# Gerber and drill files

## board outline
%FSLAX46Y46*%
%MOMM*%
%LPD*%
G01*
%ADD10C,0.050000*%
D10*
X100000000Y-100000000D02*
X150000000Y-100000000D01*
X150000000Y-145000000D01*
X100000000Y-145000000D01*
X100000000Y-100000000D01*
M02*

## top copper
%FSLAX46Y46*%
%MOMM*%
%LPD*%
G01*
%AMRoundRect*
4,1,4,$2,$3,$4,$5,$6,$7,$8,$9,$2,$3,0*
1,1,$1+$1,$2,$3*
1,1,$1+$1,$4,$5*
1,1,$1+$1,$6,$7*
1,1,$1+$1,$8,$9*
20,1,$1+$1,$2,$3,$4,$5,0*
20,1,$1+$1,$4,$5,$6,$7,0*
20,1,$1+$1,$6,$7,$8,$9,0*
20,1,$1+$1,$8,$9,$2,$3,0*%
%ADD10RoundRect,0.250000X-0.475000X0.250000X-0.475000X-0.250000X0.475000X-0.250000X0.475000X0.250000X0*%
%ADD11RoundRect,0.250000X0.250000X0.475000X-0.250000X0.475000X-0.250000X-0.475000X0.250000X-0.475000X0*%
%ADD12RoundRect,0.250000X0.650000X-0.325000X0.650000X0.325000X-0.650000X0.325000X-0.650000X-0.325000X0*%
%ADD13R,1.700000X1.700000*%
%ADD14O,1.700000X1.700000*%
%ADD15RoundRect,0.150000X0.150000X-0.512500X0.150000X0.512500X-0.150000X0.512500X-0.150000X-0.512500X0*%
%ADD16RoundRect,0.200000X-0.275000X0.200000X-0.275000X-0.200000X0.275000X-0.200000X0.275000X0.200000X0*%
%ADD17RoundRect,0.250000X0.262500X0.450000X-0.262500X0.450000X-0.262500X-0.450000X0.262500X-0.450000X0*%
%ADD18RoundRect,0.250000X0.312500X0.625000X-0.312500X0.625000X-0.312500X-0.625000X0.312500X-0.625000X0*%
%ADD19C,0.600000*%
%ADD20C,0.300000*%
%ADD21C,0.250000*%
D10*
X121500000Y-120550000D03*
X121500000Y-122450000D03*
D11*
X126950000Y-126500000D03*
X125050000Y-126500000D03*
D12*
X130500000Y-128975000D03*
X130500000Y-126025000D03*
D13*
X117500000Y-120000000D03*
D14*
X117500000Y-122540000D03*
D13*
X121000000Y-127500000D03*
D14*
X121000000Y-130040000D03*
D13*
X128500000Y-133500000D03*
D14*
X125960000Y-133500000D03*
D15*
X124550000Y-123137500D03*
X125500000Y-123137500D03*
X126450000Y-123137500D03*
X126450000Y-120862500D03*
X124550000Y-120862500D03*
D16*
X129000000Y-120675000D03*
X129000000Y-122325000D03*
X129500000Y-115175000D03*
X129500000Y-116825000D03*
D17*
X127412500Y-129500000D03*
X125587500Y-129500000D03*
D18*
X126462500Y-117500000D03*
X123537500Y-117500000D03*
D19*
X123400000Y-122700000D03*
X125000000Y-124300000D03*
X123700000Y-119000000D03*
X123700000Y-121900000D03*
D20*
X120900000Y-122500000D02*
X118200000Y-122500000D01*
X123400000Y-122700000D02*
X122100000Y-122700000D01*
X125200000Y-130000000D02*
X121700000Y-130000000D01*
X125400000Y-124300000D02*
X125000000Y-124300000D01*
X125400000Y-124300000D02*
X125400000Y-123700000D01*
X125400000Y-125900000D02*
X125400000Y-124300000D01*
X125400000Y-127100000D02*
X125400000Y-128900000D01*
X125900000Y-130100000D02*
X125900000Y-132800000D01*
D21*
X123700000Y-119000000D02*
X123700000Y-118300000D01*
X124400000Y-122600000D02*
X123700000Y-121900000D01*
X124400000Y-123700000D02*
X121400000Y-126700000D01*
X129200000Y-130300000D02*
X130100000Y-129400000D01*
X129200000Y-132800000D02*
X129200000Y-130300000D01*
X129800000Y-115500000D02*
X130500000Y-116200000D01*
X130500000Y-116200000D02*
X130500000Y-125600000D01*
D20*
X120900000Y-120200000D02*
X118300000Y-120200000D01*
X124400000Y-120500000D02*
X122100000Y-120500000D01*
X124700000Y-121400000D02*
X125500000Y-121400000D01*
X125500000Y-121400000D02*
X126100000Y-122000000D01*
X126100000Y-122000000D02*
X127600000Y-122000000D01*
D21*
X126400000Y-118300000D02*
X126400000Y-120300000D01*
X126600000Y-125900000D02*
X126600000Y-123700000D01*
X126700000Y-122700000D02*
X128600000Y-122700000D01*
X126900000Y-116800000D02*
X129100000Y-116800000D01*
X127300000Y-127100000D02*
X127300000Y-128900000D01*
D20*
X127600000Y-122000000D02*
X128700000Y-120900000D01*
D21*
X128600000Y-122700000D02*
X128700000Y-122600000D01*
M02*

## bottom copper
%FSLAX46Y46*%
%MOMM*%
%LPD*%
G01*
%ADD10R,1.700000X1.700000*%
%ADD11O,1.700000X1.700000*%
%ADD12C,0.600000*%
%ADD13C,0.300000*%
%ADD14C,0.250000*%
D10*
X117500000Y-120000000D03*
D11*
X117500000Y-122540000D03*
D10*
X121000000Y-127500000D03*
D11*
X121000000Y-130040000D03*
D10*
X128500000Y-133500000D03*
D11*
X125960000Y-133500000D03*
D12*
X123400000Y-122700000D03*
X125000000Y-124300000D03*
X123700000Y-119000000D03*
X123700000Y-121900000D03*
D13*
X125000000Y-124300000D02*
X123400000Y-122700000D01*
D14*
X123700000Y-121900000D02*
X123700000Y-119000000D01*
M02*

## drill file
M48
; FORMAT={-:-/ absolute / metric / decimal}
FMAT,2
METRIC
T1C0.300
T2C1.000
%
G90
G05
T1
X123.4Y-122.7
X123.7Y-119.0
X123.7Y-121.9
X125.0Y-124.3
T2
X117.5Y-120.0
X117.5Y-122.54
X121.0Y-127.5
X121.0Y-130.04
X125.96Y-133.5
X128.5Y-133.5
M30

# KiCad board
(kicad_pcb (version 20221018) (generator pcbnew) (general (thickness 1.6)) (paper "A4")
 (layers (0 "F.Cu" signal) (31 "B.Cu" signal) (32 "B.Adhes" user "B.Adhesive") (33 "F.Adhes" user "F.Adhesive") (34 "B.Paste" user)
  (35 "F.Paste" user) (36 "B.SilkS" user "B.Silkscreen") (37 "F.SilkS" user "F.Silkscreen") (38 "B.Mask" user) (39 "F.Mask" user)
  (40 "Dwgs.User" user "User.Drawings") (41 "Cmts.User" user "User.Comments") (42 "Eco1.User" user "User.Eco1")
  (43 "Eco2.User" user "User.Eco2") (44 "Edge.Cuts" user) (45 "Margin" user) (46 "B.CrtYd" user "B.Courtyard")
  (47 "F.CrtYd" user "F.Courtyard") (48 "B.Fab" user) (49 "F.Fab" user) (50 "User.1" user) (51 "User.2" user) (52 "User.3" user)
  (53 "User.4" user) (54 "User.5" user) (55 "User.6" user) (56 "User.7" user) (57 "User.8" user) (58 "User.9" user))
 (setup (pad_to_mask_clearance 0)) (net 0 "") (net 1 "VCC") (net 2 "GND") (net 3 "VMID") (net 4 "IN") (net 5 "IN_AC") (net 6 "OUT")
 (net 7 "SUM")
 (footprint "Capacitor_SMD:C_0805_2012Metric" (layer "F.Cu") (at 121.5 121.5 -90)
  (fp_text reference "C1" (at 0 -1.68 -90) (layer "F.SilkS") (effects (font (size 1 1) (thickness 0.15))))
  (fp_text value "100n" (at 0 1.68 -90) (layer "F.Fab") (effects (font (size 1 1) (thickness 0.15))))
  (pad "1" smd roundrect (at -0.95 0 270) (size 1 1.45) (layers "F.Cu" "F.Paste" "F.Mask") (roundrect_rratio 0.25) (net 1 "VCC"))
  (pad "2" smd roundrect (at 0.95 0 270) (size 1 1.45) (layers "F.Cu" "F.Paste" "F.Mask") (roundrect_rratio 0.25) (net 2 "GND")))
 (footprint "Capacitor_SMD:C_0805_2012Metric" (layer "F.Cu") (at 126 126.5 180)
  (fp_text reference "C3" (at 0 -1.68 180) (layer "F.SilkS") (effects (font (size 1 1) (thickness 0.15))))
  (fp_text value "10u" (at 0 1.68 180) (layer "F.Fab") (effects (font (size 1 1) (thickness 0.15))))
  (pad "1" smd roundrect (at -0.95 0 180) (size 1 1.45) (layers "F.Cu" "F.Paste" "F.Mask") (roundrect_rratio 0.25) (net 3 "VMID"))
  (pad "2" smd roundrect (at 0.95 0 180) (size 1 1.45) (layers "F.Cu" "F.Paste" "F.Mask") (roundrect_rratio 0.25) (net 2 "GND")))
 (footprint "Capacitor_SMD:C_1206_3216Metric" (layer "F.Cu") (at 130.5 127.5 90)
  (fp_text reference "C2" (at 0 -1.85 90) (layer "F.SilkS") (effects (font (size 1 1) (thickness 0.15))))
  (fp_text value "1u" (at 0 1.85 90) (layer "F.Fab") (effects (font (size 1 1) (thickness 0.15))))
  (pad "1" smd roundrect (at -1.475 0 90) (size 1.15 1.8) (layers "F.Cu" "F.Paste" "F.Mask") (roundrect_rratio 0.217391) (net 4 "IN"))
  (pad "2" smd roundrect (at 1.475 0 90) (size 1.15 1.8) (layers "F.Cu" "F.Paste" "F.Mask") (roundrect_rratio 0.217391) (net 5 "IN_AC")))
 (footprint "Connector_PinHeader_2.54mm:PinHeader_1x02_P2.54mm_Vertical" (layer "F.Cu") (at 117.5 120)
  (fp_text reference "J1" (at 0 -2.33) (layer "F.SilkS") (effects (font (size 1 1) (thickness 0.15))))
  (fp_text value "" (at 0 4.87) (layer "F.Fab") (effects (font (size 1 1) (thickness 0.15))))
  (pad "1" thru_hole rect (at 0 0) (size 1.7 1.7) (drill 1) (layers "*.Cu" "*.Mask") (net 1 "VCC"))
  (pad "2" thru_hole oval (at 0 2.54) (size 1.7 1.7) (drill 1) (layers "*.Cu" "*.Mask") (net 2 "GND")))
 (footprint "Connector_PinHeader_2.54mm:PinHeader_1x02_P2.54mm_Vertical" (layer "F.Cu") (at 121 127.5)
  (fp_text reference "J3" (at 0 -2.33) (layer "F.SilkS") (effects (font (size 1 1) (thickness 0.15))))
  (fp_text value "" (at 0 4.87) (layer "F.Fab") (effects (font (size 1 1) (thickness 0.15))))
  (pad "1" thru_hole rect (at 0 0) (size 1.7 1.7) (drill 1) (layers "*.Cu" "*.Mask") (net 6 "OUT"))
  (pad "2" thru_hole oval (at 0 2.54) (size 1.7 1.7) (drill 1) (layers "*.Cu" "*.Mask") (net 2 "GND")))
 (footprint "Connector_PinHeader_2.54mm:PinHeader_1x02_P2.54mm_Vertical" (layer "F.Cu") (at 128.5 133.5 -90)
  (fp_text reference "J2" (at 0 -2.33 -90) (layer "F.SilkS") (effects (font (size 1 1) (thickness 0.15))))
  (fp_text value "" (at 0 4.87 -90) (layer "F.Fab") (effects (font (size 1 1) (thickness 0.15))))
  (pad "1" thru_hole rect (at 0 0 270) (size 1.7 1.7) (drill 1) (layers "*.Cu" "*.Mask") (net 4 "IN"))
  (pad "2" thru_hole oval (at 0 2.54 270) (size 1.7 1.7) (drill 1) (layers "*.Cu" "*.Mask") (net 2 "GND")))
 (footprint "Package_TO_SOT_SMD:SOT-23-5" (layer "F.Cu") (at 125.5 122 90)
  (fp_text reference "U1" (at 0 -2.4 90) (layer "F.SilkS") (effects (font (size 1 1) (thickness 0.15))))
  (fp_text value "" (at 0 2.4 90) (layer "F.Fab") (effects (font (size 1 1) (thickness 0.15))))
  (pad "1" smd roundrect (at -1.1375 -0.95 90) (size 1.325 0.6) (layers "F.Cu" "F.Paste" "F.Mask") (roundrect_rratio 0.25) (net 6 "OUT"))
  (pad "2" smd roundrect (at -1.1375 0 90) (size 1.325 0.6) (layers "F.Cu" "F.Paste" "F.Mask") (roundrect_rratio 0.25) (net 2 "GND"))
  (pad "3" smd roundrect (at -1.1375 0.95 90) (size 1.325 0.6) (layers "F.Cu" "F.Paste" "F.Mask") (roundrect_rratio 0.25) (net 3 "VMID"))
  (pad "4" smd roundrect (at 1.1375 0.95 90) (size 1.325 0.6) (layers "F.Cu" "F.Paste" "F.Mask") (roundrect_rratio 0.25) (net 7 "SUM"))
  (pad "5" smd roundrect (at 1.1375 -0.95 90) (size 1.325 0.6) (layers "F.Cu" "F.Paste" "F.Mask") (roundrect_rratio 0.25) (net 1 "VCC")))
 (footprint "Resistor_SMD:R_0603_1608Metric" (layer "F.Cu") (at 129 121.5 -90)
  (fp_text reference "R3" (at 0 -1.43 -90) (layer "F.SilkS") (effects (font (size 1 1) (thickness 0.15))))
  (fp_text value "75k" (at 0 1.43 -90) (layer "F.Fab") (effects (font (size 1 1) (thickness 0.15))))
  (pad "1" smd roundrect (at -0.825 0 270) (size 0.8 0.95) (layers "F.Cu" "F.Paste" "F.Mask") (roundrect_rratio 0.25) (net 1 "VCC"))
  (pad "2" smd roundrect (at 0.825 0 270) (size 0.8 0.95) (layers "F.Cu" "F.Paste" "F.Mask") (roundrect_rratio 0.25) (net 3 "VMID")))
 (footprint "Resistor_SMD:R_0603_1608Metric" (layer "F.Cu") (at 129.5 116 -90)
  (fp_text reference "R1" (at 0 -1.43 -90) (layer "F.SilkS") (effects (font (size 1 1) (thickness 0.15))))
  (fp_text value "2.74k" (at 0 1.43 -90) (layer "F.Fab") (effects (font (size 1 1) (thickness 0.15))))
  (pad "1" smd roundrect (at -0.825 0 270) (size 0.8 0.95) (layers "F.Cu" "F.Paste" "F.Mask") (roundrect_rratio 0.25) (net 5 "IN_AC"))
  (pad "2" smd roundrect (at 0.825 0 270) (size 0.8 0.95) (layers "F.Cu" "F.Paste" "F.Mask") (roundrect_rratio 0.25) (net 7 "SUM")))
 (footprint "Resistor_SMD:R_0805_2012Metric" (layer "F.Cu") (at 126.5 129.5 180)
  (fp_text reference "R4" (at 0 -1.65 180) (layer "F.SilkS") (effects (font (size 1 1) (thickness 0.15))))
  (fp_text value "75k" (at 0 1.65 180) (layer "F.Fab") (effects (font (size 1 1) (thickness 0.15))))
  (pad "1" smd roundrect (at -0.9125 0 180) (size 1.025 1.4) (layers "F.Cu" "F.Paste" "F.Mask") (roundrect_rratio 0.243902) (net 3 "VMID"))
  (pad "2" smd roundrect (at 0.9125 0 180) (size 1.025 1.4) (layers "F.Cu" "F.Paste" "F.Mask") (roundrect_rratio 0.243902) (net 2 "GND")))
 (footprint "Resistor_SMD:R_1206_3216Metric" (layer "F.Cu") (at 125 117.5 180)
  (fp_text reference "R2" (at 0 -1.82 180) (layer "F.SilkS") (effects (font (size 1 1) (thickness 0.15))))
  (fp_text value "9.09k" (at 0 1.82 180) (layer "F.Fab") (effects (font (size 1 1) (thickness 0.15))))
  (pad "1" smd roundrect (at -1.4625 0 180) (size 1.125 1.75) (layers "F.Cu" "F.Paste" "F.Mask") (roundrect_rratio 0.222222) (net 7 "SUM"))
  (pad "2" smd roundrect (at 1.4625 0 180) (size 1.125 1.75) (layers "F.Cu" "F.Paste" "F.Mask") (roundrect_rratio 0.222222) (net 6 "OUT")))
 (gr_rect (start 100 100) (end 150 145) (stroke (width 0.05) (type default)) (fill none) (layer "Edge.Cuts"))
 (segment (start 120.9 122.5) (end 118.2 122.5) (width 0.3) (layer "F.Cu") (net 2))
 (segment (start 123.4 122.7) (end 122.1 122.7) (width 0.3) (layer "F.Cu") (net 2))
 (segment (start 125.2 130) (end 121.7 130) (width 0.3) (layer "F.Cu") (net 2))
 (segment (start 125.4 124.3) (end 125 124.3) (width 0.3) (layer "F.Cu") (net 2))
 (segment (start 125.4 124.3) (end 125.4 123.7) (width 0.3) (layer "F.Cu") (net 2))
 (segment (start 125.4 125.9) (end 125.4 124.3) (width 0.3) (layer "F.Cu") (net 2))
 (segment (start 125.4 127.1) (end 125.4 128.9) (width 0.3) (layer "F.Cu") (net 2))
 (segment (start 125.9 130.1) (end 125.9 132.8) (width 0.3) (layer "F.Cu") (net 2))
 (via (at 123.4 122.7) (size 0.6) (drill 0.3) (layers "F.Cu" "B.Cu") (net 2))
 (via (at 125 124.3) (size 0.6) (drill 0.3) (layers "F.Cu" "B.Cu") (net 2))
 (segment (start 123.7 119) (end 123.7 118.3) (width 0.25) (layer "F.Cu") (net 6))
 (segment (start 124.4 122.6) (end 123.7 121.9) (width 0.25) (layer "F.Cu") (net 6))
 (segment (start 124.4 123.7) (end 121.4 126.7) (width 0.25) (layer "F.Cu") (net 6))
 (segment (start 125 124.3) (end 123.4 122.7) (width 0.3) (layer "B.Cu") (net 2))
 (segment (start 129.2 130.3) (end 130.1 129.4) (width 0.25) (layer "F.Cu") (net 4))
 (segment (start 129.2 132.8) (end 129.2 130.3) (width 0.25) (layer "F.Cu") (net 4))
 (segment (start 129.8 115.5) (end 130.5 116.2) (width 0.25) (layer "F.Cu") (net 5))
 (segment (start 130.5 116.2) (end 130.5 125.6) (width 0.25) (layer "F.Cu") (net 5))
 (via (at 123.7 119) (size 0.6) (drill 0.3) (layers "F.Cu" "B.Cu") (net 6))
 (via (at 123.7 121.9) (size 0.6) (drill 0.3) (layers "F.Cu" "B.Cu") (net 6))
 (segment (start 120.9 120.2) (end 118.3 120.2) (width 0.3) (layer "F.Cu") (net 1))
 (segment (start 123.7 121.9) (end 123.7 119) (width 0.25) (layer "B.Cu") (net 6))
 (segment (start 124.4 120.5) (end 122.1 120.5) (width 0.3) (layer "F.Cu") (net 1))
 (segment (start 124.7 121.4) (end 125.5 121.4) (width 0.3) (layer "F.Cu") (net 1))
 (segment (start 125.5 121.4) (end 126.1 122) (width 0.3) (layer "F.Cu") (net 1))
 (segment (start 126.1 122) (end 127.6 122) (width 0.3) (layer "F.Cu") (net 1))
 (segment (start 126.4 118.3) (end 126.4 120.3) (width 0.25) (layer "F.Cu") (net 7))
 (segment (start 126.6 125.9) (end 126.6 123.7) (width 0.25) (layer "F.Cu") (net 3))
 (segment (start 126.7 122.7) (end 128.6 122.7) (width 0.25) (layer "F.Cu") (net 3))
 (segment (start 126.9 116.8) (end 129.1 116.8) (width 0.25) (layer "F.Cu") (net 7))
 (segment (start 127.3 127.1) (end 127.3 128.9) (width 0.25) (layer "F.Cu") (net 3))
 (segment (start 127.6 122) (end 128.7 120.9) (width 0.3) (layer "F.Cu") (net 1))
 (segment (start 128.6 122.7) (end 128.7 122.6) (width 0.25) (layer "F.Cu") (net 3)))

